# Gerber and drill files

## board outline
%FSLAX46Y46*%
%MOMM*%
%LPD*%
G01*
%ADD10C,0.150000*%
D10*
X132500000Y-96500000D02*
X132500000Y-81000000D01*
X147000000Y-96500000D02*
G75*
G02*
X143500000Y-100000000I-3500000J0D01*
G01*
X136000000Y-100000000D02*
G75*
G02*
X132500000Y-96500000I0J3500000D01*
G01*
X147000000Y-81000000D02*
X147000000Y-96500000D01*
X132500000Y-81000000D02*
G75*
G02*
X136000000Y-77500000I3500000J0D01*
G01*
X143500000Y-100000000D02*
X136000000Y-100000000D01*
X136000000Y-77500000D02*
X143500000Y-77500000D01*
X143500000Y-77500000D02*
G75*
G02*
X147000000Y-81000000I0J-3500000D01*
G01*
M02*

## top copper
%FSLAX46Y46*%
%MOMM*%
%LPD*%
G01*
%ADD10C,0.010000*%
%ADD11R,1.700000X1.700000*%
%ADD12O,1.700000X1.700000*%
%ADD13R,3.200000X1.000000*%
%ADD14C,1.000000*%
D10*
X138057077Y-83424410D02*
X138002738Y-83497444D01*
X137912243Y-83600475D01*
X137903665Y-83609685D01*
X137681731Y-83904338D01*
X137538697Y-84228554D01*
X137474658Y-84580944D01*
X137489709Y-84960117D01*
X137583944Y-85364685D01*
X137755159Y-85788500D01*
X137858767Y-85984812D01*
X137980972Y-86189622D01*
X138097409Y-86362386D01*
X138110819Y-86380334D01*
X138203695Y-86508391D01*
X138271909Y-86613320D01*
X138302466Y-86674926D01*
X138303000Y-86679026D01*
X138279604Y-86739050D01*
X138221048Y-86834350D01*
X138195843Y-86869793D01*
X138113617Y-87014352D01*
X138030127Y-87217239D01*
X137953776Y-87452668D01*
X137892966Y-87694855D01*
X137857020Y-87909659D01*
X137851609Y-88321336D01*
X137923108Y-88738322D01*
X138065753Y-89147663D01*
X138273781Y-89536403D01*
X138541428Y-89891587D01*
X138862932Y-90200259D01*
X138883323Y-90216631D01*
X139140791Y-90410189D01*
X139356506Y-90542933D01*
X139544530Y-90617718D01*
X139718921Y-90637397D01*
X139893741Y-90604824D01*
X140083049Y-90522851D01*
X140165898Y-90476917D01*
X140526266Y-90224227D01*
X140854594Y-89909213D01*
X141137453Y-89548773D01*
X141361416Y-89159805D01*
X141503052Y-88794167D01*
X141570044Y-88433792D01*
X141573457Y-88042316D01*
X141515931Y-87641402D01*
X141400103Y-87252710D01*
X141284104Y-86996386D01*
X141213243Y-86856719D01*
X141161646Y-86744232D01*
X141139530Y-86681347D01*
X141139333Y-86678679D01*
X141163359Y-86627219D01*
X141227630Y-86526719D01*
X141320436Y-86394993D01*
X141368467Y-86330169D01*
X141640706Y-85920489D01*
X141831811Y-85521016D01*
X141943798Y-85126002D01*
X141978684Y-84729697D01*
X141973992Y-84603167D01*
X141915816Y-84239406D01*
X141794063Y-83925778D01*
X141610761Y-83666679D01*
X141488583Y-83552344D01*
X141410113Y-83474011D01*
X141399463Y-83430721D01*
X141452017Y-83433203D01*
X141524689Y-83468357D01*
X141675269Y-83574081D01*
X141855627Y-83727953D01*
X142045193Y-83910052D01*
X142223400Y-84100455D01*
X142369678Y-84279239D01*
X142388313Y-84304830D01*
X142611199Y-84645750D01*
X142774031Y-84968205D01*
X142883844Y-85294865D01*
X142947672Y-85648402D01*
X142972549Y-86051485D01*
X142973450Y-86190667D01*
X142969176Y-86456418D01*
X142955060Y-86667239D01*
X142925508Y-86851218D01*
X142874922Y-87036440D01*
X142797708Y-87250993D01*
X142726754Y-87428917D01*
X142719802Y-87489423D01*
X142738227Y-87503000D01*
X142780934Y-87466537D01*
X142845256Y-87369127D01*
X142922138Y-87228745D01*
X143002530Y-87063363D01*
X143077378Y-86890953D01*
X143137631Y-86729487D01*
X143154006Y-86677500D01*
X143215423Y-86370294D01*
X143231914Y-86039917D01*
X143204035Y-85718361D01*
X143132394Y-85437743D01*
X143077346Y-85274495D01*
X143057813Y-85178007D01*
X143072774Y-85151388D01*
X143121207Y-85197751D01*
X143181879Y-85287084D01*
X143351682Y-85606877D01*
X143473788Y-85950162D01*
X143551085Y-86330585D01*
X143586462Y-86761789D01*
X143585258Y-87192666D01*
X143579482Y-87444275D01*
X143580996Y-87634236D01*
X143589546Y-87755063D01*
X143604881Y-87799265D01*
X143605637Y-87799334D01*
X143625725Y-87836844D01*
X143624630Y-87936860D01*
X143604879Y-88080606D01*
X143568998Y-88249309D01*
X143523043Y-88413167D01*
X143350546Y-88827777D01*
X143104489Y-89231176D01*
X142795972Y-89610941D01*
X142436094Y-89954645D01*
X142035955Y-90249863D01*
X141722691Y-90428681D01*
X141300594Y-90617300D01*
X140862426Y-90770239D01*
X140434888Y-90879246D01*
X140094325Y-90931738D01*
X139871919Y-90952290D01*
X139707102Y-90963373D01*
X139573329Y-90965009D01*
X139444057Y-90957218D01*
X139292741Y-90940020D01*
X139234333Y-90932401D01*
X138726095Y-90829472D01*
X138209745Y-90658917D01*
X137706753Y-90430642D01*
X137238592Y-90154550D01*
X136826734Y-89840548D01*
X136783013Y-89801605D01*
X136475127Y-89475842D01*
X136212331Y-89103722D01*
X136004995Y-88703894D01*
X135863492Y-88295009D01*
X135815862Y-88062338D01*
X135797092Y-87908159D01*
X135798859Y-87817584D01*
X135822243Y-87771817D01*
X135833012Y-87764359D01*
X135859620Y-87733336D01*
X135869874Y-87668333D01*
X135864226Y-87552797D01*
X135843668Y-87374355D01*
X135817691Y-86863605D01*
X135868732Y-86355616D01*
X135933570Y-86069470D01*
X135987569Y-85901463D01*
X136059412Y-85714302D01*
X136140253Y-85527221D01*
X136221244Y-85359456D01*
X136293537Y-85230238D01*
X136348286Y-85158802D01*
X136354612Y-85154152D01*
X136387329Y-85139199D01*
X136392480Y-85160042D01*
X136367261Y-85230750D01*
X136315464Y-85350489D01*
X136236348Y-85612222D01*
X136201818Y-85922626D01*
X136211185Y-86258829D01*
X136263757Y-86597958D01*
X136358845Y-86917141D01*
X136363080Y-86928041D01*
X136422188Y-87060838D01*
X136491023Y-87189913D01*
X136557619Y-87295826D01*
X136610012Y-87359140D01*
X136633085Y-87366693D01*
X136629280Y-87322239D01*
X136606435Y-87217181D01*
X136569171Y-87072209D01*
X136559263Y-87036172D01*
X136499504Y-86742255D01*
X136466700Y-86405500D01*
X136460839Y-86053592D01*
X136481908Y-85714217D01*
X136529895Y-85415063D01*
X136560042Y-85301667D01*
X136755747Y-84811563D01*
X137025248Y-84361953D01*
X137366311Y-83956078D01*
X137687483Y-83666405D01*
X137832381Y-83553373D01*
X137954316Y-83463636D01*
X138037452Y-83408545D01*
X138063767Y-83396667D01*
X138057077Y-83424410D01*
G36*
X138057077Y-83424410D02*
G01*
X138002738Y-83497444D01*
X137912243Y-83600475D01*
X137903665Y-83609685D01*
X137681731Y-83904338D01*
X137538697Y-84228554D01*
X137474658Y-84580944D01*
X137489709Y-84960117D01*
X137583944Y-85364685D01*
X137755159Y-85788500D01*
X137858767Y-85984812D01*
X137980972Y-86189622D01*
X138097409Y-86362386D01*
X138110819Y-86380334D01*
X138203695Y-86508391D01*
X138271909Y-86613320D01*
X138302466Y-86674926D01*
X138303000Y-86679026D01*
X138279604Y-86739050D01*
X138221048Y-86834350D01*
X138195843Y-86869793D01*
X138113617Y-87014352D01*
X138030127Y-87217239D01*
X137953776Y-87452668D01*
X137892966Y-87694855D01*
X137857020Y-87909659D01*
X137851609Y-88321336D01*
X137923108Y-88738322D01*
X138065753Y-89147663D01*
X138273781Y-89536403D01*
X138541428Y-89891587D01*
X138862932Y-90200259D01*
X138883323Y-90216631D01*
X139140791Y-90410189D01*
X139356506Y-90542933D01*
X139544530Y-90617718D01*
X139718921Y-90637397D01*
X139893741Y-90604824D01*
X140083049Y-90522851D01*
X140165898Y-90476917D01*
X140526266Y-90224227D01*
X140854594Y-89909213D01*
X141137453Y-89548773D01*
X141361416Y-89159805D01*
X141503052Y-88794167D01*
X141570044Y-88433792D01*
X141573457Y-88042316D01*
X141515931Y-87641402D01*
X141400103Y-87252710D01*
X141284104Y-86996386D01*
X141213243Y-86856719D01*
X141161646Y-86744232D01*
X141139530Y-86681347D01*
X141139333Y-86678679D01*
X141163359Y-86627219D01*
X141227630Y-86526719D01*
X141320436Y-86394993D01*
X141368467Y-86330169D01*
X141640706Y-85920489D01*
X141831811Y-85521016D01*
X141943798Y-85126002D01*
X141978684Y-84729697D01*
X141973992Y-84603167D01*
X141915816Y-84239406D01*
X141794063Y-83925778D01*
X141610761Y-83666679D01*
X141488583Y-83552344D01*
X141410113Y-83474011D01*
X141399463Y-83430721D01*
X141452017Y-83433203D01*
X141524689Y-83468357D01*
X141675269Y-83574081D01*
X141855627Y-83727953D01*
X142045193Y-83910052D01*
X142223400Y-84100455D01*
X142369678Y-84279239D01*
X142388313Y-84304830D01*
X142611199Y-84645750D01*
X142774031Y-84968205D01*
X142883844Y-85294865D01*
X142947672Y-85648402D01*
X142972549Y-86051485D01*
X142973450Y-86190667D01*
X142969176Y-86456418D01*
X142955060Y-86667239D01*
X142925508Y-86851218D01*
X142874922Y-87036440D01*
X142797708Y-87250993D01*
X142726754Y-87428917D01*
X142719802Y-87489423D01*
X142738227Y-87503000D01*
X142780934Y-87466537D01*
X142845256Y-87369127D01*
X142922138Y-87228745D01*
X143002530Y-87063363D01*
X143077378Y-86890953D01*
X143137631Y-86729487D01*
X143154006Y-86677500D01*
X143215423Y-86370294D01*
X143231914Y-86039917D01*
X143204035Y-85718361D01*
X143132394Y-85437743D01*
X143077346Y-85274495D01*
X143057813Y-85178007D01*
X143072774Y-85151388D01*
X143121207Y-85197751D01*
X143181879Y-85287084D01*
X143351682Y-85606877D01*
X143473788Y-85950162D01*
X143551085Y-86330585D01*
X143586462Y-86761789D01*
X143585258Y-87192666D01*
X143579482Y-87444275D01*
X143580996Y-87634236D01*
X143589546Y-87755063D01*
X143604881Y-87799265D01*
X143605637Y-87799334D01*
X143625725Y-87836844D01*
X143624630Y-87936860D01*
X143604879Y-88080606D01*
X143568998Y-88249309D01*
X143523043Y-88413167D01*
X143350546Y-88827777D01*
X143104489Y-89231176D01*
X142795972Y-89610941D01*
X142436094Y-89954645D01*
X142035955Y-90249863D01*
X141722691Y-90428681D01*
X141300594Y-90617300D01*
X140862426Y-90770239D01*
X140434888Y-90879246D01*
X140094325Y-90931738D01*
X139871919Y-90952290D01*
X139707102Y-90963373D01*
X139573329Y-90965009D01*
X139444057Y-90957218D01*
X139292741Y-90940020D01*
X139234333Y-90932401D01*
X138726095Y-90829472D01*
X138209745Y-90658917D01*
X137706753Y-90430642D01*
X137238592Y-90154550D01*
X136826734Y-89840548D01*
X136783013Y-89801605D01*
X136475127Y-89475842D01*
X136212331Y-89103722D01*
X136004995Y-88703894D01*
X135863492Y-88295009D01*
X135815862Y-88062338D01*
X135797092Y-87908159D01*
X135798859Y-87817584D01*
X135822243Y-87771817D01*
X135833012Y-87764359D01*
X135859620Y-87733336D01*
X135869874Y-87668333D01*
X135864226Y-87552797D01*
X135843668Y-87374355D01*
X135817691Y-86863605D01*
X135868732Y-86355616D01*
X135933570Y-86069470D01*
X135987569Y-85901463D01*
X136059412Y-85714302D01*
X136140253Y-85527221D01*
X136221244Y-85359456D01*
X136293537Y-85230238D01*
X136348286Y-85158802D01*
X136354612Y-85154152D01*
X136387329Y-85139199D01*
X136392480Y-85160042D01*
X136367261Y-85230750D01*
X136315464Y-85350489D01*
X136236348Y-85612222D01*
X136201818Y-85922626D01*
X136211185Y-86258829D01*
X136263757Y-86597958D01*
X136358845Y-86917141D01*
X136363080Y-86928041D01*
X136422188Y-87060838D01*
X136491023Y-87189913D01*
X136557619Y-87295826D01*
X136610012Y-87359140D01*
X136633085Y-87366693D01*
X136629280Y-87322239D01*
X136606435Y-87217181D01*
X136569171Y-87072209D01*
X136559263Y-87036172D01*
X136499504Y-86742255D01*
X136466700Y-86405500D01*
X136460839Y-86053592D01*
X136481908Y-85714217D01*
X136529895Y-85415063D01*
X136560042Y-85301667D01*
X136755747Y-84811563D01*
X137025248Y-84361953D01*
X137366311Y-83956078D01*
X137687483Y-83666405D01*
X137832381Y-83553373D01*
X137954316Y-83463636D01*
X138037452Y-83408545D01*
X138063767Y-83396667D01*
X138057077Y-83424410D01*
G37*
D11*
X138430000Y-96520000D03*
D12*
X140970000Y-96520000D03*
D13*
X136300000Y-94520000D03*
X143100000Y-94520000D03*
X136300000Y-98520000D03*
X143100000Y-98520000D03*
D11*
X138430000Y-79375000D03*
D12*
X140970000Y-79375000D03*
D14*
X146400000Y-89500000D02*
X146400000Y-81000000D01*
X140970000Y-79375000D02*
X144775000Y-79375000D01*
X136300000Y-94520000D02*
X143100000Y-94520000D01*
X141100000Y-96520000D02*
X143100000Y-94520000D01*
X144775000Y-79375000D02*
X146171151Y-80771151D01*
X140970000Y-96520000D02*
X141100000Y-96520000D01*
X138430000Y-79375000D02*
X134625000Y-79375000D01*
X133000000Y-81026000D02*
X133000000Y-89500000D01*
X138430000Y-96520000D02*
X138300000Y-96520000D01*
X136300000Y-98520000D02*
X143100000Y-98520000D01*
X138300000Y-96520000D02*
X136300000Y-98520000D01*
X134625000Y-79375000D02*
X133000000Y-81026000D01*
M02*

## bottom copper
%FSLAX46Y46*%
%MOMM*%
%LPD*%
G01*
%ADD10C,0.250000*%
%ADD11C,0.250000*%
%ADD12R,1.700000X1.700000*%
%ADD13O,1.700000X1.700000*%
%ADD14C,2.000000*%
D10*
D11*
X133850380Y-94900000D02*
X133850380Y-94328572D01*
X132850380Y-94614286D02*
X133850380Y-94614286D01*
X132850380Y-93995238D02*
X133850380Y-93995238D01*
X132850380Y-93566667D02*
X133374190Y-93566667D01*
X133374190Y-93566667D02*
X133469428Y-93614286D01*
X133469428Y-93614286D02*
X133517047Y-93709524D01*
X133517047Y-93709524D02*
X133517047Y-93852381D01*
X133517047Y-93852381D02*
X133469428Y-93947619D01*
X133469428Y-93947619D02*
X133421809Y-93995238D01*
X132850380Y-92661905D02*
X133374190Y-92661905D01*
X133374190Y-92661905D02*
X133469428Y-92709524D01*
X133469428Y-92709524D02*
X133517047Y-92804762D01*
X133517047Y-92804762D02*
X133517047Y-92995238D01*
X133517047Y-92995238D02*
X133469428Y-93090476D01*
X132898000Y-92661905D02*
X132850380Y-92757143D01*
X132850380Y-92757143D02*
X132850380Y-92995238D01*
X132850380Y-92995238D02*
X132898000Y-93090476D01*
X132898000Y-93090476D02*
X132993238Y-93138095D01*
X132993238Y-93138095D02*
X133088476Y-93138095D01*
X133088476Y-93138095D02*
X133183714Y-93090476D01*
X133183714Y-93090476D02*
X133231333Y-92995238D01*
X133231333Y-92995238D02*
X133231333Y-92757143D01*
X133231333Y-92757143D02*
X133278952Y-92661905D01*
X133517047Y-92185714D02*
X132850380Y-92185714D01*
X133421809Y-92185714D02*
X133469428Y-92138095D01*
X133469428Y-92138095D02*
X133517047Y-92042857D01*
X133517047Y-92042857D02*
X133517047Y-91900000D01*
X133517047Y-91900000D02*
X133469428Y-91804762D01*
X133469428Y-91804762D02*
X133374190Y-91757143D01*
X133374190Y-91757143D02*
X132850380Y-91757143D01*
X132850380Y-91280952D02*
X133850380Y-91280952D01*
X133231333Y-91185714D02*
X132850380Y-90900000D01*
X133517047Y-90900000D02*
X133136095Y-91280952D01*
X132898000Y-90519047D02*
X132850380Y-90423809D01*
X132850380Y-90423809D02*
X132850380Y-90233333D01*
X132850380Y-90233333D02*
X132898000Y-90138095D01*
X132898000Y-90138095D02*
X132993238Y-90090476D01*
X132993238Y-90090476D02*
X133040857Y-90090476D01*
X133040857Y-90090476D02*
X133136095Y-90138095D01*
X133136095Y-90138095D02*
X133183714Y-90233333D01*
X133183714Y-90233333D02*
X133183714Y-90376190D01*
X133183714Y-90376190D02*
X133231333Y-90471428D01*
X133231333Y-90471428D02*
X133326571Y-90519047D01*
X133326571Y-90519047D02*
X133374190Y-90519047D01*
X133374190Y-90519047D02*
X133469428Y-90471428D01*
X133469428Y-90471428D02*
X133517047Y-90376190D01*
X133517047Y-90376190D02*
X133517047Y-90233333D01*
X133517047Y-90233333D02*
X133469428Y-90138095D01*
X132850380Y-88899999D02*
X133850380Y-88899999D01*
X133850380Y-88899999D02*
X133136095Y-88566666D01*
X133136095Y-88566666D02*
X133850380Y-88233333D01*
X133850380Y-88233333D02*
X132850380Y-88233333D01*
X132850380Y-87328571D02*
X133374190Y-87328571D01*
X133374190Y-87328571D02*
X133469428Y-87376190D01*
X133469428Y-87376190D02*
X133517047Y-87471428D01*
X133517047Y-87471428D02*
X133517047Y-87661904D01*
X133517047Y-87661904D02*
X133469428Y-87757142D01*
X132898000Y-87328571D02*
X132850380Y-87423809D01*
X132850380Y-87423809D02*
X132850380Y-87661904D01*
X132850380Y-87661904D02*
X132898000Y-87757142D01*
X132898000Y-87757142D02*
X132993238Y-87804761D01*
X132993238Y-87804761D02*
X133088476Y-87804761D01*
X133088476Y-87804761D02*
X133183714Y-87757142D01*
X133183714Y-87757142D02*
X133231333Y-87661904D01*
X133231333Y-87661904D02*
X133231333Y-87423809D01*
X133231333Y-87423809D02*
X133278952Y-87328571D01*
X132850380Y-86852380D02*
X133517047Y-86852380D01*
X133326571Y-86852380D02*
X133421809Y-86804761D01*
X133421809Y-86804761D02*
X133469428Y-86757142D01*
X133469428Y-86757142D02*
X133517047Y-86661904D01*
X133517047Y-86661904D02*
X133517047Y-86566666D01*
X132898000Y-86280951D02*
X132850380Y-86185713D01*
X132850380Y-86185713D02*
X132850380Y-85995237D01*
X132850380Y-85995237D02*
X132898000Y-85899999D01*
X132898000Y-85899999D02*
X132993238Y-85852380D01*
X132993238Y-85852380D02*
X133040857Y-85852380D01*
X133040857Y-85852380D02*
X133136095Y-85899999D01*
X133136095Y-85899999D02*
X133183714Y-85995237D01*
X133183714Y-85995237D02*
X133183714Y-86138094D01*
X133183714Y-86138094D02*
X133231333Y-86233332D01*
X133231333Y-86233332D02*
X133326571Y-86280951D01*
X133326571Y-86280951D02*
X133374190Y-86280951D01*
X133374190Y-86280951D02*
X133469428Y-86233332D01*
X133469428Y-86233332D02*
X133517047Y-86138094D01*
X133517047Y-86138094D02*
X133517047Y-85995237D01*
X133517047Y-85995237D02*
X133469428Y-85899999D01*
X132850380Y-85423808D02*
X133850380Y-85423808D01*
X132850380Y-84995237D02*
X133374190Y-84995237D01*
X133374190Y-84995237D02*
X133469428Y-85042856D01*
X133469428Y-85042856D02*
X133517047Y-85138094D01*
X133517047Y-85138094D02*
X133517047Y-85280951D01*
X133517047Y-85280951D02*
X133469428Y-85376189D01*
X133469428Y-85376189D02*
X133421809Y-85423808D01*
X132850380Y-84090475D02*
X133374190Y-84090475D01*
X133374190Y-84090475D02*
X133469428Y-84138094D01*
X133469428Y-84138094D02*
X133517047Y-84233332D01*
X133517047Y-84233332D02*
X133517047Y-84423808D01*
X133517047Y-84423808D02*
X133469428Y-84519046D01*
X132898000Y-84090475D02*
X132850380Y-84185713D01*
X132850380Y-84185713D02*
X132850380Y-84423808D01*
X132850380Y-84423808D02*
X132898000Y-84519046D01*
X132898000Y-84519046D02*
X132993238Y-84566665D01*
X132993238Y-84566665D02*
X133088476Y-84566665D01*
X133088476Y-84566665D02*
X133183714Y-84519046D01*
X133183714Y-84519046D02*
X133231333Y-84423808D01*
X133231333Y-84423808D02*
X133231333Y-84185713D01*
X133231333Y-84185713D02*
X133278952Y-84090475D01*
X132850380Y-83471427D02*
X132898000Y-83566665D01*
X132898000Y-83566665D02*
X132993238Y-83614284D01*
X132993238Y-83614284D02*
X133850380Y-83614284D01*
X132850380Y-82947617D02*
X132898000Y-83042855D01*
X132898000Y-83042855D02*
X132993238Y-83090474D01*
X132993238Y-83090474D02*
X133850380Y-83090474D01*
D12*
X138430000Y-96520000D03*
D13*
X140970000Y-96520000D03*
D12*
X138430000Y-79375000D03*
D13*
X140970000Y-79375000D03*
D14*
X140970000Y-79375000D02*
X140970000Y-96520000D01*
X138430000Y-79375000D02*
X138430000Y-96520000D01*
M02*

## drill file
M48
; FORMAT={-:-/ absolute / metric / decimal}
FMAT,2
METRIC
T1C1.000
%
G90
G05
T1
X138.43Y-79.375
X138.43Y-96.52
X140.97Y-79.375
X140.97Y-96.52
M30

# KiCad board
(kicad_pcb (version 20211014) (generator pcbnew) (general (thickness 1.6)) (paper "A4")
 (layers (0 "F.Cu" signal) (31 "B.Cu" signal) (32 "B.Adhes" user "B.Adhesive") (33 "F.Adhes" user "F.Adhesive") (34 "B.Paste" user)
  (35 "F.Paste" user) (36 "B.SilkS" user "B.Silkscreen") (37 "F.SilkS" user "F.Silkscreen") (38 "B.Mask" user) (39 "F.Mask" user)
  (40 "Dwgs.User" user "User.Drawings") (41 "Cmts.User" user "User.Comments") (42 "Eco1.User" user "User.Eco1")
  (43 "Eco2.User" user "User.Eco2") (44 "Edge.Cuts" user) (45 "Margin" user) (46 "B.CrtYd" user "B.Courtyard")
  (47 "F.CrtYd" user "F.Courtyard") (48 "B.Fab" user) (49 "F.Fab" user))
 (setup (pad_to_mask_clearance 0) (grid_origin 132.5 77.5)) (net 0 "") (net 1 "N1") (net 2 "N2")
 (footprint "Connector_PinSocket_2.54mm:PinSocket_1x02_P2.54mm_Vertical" (layer "F.Cu") (at 138.43 96.52 90)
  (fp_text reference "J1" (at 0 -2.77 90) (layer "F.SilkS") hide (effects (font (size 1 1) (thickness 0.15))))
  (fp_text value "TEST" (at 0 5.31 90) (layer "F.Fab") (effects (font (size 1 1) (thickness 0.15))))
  (pad "1" thru_hole rect locked (at 0 0 90) (size 1.7 1.7) (drill 1) (layers *.Cu *.Mask) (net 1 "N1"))
  (pad "2" thru_hole oval locked (at 0 2.54 90) (size 1.7 1.7) (drill 1) (layers *.Cu *.Mask) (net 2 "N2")))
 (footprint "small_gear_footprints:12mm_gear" (layer "F.Cu") (at 139.7 86.995)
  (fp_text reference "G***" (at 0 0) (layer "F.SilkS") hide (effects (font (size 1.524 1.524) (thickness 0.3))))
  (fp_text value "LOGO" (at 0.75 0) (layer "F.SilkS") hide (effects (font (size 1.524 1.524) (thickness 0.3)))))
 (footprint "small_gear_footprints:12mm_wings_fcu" (layer "F.Cu") (at 139.7 86.995)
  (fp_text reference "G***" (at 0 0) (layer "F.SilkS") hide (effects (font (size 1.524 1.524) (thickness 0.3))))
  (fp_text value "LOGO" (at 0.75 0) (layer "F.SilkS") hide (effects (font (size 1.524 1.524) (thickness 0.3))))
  (fp_poly
   (pts (xy -1.642923 -3.57059) (xy -1.697262 -3.497556) (xy -1.787757 -3.394525) (xy -1.796335 -3.385315) (xy -2.018269 -3.090662)
    (xy -2.161303 -2.766446) (xy -2.225342 -2.414056) (xy -2.210291 -2.034883) (xy -2.116056 -1.630315) (xy -1.944841 -1.2065)
    (xy -1.841233 -1.010188) (xy -1.719028 -0.805378) (xy -1.602591 -0.632614) (xy -1.589181 -0.614666) (xy -1.496305 -0.486609)
    (xy -1.428091 -0.38168) (xy -1.397534 -0.320074) (xy -1.397 -0.315974) (xy -1.420396 -0.25595) (xy -1.478952 -0.16065)
    (xy -1.504157 -0.125207) (xy -1.586383 0.019352) (xy -1.669873 0.222239) (xy -1.746224 0.457668) (xy -1.807034 0.699855)
    (xy -1.84298 0.914659) (xy -1.848391 1.326336) (xy -1.776892 1.743322) (xy -1.634247 2.152663) (xy -1.426219 2.541403)
    (xy -1.158572 2.896587) (xy -0.837068 3.205259) (xy -0.816677 3.221631) (xy -0.559209 3.415189) (xy -0.343494 3.547933)
    (xy -0.15547 3.622718) (xy 0.018921 3.642397) (xy 0.193741 3.609824) (xy 0.383049 3.527851) (xy 0.465898 3.481917)
    (xy 0.826266 3.229227) (xy 1.154594 2.914213) (xy 1.437453 2.553773) (xy 1.661416 2.164805) (xy 1.803052 1.799167)
    (xy 1.870044 1.438792) (xy 1.873457 1.047316) (xy 1.815931 0.646402) (xy 1.700103 0.25771) (xy 1.584104 0.001386)
    (xy 1.513243 -0.138281) (xy 1.461646 -0.250768) (xy 1.43953 -0.313653) (xy 1.439333 -0.316321) (xy 1.463359 -0.367781)
    (xy 1.52763 -0.468281) (xy 1.620436 -0.600007) (xy 1.668467 -0.664831) (xy 1.940706 -1.074511) (xy 2.131811 -1.473984)
    (xy 2.243798 -1.868998) (xy 2.278684 -2.265303) (xy 2.273992 -2.391833) (xy 2.215816 -2.755594) (xy 2.094063 -3.069222)
    (xy 1.910761 -3.328321) (xy 1.788583 -3.442656) (xy 1.710113 -3.520989) (xy 1.699463 -3.564279) (xy 1.752017 -3.561797)
    (xy 1.824689 -3.526643) (xy 1.975269 -3.420919) (xy 2.155627 -3.267047) (xy 2.345193 -3.084948) (xy 2.5234 -2.894545)
    (xy 2.669678 -2.715761) (xy 2.688313 -2.69017) (xy 2.911199 -2.34925) (xy 3.074031 -2.026795) (xy 3.183844 -1.700135)
    (xy 3.247672 -1.346598) (xy 3.272549 -0.943515) (xy 3.27345 -0.804333) (xy 3.269176 -0.538582) (xy 3.25506 -0.327761)
    (xy 3.225508 -0.143782) (xy 3.174922 0.04144) (xy 3.097708 0.255993) (xy 3.026754 0.433917) (xy 3.019802 0.494423) (xy 3.038227 0.508)
    (xy 3.080934 0.471537) (xy 3.145256 0.374127) (xy 3.222138 0.233745) (xy 3.30253 0.068363) (xy 3.377378 -0.104047)
    (xy 3.437631 -0.265513) (xy 3.454006 -0.3175) (xy 3.515423 -0.624706) (xy 3.531914 -0.955083) (xy 3.504035 -1.276639)
    (xy 3.432394 -1.557257) (xy 3.377346 -1.720505) (xy 3.357813 -1.816993) (xy 3.372774 -1.843612) (xy 3.421207 -1.797249)
    (xy 3.481879 -1.707916) (xy 3.651682 -1.388123) (xy 3.773788 -1.044838) (xy 3.851085 -0.664415) (xy 3.886462 -0.233211)
    (xy 3.885258 0.197666) (xy 3.879482 0.449275) (xy 3.880996 0.639236) (xy 3.889546 0.760063) (xy 3.904881 0.804265)
    (xy 3.905637 0.804334) (xy 3.925725 0.841844) (xy 3.92463 0.94186) (xy 3.904879 1.085606) (xy 3.868998 1.254309) (xy 3.823043 1.418167)
    (xy 3.650546 1.832777) (xy 3.404489 2.236176) (xy 3.095972 2.615941) (xy 2.736094 2.959645) (xy 2.335955 3.254863)
    (xy 2.022691 3.433681) (xy 1.600594 3.6223) (xy 1.162426 3.775239) (xy 0.734888 3.884246) (xy 0.394325 3.936738) (xy 0.171919 3.95729)
    (xy 0.007102 3.968373) (xy -0.126671 3.970009) (xy -0.255943 3.962218) (xy -0.407259 3.94502) (xy -0.465667 3.937401)
    (xy -0.973905 3.834472) (xy -1.490255 3.663917) (xy -1.993247 3.435642) (xy -2.461408 3.15955) (xy -2.873266 2.845548)
    (xy -2.916987 2.806605) (xy -3.224873 2.480842) (xy -3.487669 2.108722) (xy -3.695005 1.708894) (xy -3.836508 1.300009)
    (xy -3.884138 1.067338) (xy -3.902908 0.913159) (xy -3.901141 0.822584) (xy -3.877757 0.776817) (xy -3.866988 0.769359)
    (xy -3.84038 0.738336) (xy -3.830126 0.673333) (xy -3.835774 0.557797) (xy -3.856332 0.379355) (xy -3.882309 -0.131395)
    (xy -3.831268 -0.639384) (xy -3.76643 -0.92553) (xy -3.712431 -1.093537) (xy -3.640588 -1.280698) (xy -3.559747 -1.467779)
    (xy -3.478756 -1.635544) (xy -3.406463 -1.764762) (xy -3.351714 -1.836198) (xy -3.345388 -1.840848) (xy -3.312671 -1.855801)
    (xy -3.30752 -1.834958) (xy -3.332739 -1.76425) (xy -3.384536 -1.644511) (xy -3.463652 -1.382778) (xy -3.498182 -1.072374)
    (xy -3.488815 -0.736171) (xy -3.436243 -0.397042) (xy -3.341155 -0.077859) (xy -3.33692 -0.066959) (xy -3.277812 0.065838)
    (xy -3.208977 0.194913) (xy -3.142381 0.300826) (xy -3.089988 0.36414) (xy -3.066915 0.371693) (xy -3.07072 0.327239)
    (xy -3.093565 0.222181) (xy -3.130829 0.077209) (xy -3.140737 0.041172) (xy -3.200496 -0.252745) (xy -3.2333 -0.5895)
    (xy -3.239161 -0.941408) (xy -3.218092 -1.280783) (xy -3.170105 -1.579937) (xy -3.139958 -1.693333) (xy -2.944253 -2.183437)
    (xy -2.674752 -2.633047) (xy -2.333689 -3.038922) (xy -2.012517 -3.328595) (xy -1.867619 -3.441627) (xy -1.745684 -3.531364)
    (xy -1.662548 -3.586455) (xy -1.636233 -3.598333) (xy -1.642923 -3.57059))
   (layer "F.Cu") (width 0.01) (fill solid)))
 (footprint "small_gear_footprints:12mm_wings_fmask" (layer "F.Cu") (at 139.7 86.995)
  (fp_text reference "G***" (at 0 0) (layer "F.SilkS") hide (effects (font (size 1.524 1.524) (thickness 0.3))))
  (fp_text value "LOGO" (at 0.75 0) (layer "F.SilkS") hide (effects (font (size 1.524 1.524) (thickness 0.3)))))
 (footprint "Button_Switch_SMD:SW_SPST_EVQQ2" (layer "F.Cu") (at 139.7 96.52)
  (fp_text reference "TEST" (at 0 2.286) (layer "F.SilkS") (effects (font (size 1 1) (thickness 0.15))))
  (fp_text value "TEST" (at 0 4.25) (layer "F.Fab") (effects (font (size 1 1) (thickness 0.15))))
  (pad "1" smd rect locked (at -3.4 -2) (size 3.2 1) (layers "F.Cu" "F.Paste" "F.Mask") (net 2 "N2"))
  (pad "1" smd rect locked (at 3.4 -2) (size 3.2 1) (layers "F.Cu" "F.Paste" "F.Mask") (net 2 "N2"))
  (pad "2" smd rect locked (at -3.4 2) (size 3.2 1) (layers "F.Cu" "F.Paste" "F.Mask") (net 1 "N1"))
  (pad "2" smd rect locked (at 3.4 2) (size 3.2 1) (layers "F.Cu" "F.Paste" "F.Mask") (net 1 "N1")))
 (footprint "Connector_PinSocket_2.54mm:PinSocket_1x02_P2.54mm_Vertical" (layer "F.Cu") (at 138.43 79.375 90)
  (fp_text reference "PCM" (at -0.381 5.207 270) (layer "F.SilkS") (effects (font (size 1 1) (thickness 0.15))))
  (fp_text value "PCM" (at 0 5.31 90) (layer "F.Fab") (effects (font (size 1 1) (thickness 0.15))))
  (pad "1" thru_hole rect locked (at 0 0 90) (size 1.7 1.7) (drill 1) (layers *.Cu *.Mask) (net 1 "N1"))
  (pad "2" thru_hole oval locked (at 0 2.54 90) (size 1.7 1.7) (drill 1) (layers *.Cu *.Mask) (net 2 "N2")))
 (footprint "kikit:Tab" (layer "F.Cu") (at 139.75 77.1 -90)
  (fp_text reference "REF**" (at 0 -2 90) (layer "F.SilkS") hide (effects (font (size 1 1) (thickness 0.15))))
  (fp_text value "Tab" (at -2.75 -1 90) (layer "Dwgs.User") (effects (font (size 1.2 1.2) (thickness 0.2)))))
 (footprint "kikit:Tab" (layer "F.Cu") (at 139.75 100.35 90)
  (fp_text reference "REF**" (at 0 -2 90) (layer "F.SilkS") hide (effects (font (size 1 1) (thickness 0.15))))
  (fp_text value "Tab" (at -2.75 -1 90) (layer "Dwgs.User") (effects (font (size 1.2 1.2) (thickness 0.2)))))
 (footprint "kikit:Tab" (layer "F.Cu") (at 132.1 95)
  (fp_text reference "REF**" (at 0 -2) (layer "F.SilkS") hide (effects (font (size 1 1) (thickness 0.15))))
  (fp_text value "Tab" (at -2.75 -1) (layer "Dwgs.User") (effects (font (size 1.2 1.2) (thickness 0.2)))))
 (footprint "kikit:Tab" (layer "F.Cu") (at 132.1 82.5)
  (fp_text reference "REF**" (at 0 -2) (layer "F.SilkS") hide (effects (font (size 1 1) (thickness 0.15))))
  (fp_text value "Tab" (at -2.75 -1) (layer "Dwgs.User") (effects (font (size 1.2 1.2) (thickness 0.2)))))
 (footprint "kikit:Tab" (layer "F.Cu") (at 147.4 95 180)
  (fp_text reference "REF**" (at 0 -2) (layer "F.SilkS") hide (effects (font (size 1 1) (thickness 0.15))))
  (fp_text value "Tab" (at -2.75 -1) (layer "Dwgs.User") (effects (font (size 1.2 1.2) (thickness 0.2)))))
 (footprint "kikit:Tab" (layer "F.Cu") (at 147.4 82.5 180)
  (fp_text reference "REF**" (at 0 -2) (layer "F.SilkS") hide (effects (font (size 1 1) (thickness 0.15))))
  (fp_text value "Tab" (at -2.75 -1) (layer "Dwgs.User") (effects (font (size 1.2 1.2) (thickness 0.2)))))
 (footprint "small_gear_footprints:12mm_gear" (layer "B.Cu") (at 139.7 86.995 180)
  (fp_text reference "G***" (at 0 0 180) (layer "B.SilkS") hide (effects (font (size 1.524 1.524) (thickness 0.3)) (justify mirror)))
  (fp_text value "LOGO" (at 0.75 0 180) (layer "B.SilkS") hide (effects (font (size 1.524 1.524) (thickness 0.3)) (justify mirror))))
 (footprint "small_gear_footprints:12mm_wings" (layer "B.Cu") (at 139.7 86.995 180)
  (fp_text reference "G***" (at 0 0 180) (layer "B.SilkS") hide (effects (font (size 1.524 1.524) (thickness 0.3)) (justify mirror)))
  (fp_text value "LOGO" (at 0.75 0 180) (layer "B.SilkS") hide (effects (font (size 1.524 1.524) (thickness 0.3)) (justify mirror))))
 (gr_line (start 132.5 96.5) (end 132.5 81) (layer "Edge.Cuts") (width 0.15))
 (gr_arc (start 147 96.5) (mid 145.974874 98.974874) (end 143.5 100) (layer "Edge.Cuts") (width 0.15))
 (gr_arc (start 136 100) (mid 133.525126 98.974874) (end 132.5 96.5) (layer "Edge.Cuts") (width 0.15))
 (gr_line (start 147 81) (end 147 96.5) (layer "Edge.Cuts") (width 0.15))
 (gr_arc (start 132.5 81) (mid 133.525126 78.525126) (end 136 77.5) (layer "Edge.Cuts") (width 0.15))
 (gr_line (start 143.5 100) (end 136 100) (layer "Edge.Cuts") (width 0.15))
 (gr_line (start 136 77.5) (end 143.5 77.5) (layer "Edge.Cuts") (width 0.15))
 (gr_arc (start 143.5 77.5) (mid 145.974874 78.525126) (end 147 81) (layer "Edge.Cuts") (width 0.15))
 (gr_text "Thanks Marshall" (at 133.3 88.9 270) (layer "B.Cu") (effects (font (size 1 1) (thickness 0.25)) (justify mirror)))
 (segment (start 146.4 89.5) (end 146.4 81) (width 1) (layer "F.Cu") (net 2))
 (segment (start 140.97 79.375) (end 144.775 79.375) (width 1) (layer "F.Cu") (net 2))
 (segment (start 136.3 94.52) (end 143.1 94.52) (width 1) (layer "F.Cu") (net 2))
 (segment (start 141.1 96.52) (end 143.1 94.52) (width 1) (layer "F.Cu") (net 2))
 (segment (start 144.775 79.375) (end 146.171151 80.771151) (width 1) (layer "F.Cu") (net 2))
 (segment (start 140.97 96.52) (end 141.1 96.52) (width 1) (layer "F.Cu") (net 2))
 (segment (start 140.97 79.375) (end 140.97 96.52) (width 2) (layer "B.Cu") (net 2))
 (segment (start 138.43 79.375) (end 134.625 79.375) (width 1) (layer "F.Cu") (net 1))
 (segment (start 133 81.026) (end 133 89.5) (width 1) (layer "F.Cu") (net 1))
 (segment (start 138.43 96.52) (end 138.3 96.52) (width 1) (layer "F.Cu") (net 1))
 (segment (start 136.3 98.52) (end 143.1 98.52) (width 1) (layer "F.Cu") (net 1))
 (segment (start 138.3 96.52) (end 136.3 98.52) (width 1) (layer "F.Cu") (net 1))
 (segment (start 134.625 79.375) (end 133 81.026) (width 1) (layer "F.Cu") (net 1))
 (segment (start 138.43 79.375) (end 138.43 96.52) (width 2) (layer "B.Cu") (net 1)))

